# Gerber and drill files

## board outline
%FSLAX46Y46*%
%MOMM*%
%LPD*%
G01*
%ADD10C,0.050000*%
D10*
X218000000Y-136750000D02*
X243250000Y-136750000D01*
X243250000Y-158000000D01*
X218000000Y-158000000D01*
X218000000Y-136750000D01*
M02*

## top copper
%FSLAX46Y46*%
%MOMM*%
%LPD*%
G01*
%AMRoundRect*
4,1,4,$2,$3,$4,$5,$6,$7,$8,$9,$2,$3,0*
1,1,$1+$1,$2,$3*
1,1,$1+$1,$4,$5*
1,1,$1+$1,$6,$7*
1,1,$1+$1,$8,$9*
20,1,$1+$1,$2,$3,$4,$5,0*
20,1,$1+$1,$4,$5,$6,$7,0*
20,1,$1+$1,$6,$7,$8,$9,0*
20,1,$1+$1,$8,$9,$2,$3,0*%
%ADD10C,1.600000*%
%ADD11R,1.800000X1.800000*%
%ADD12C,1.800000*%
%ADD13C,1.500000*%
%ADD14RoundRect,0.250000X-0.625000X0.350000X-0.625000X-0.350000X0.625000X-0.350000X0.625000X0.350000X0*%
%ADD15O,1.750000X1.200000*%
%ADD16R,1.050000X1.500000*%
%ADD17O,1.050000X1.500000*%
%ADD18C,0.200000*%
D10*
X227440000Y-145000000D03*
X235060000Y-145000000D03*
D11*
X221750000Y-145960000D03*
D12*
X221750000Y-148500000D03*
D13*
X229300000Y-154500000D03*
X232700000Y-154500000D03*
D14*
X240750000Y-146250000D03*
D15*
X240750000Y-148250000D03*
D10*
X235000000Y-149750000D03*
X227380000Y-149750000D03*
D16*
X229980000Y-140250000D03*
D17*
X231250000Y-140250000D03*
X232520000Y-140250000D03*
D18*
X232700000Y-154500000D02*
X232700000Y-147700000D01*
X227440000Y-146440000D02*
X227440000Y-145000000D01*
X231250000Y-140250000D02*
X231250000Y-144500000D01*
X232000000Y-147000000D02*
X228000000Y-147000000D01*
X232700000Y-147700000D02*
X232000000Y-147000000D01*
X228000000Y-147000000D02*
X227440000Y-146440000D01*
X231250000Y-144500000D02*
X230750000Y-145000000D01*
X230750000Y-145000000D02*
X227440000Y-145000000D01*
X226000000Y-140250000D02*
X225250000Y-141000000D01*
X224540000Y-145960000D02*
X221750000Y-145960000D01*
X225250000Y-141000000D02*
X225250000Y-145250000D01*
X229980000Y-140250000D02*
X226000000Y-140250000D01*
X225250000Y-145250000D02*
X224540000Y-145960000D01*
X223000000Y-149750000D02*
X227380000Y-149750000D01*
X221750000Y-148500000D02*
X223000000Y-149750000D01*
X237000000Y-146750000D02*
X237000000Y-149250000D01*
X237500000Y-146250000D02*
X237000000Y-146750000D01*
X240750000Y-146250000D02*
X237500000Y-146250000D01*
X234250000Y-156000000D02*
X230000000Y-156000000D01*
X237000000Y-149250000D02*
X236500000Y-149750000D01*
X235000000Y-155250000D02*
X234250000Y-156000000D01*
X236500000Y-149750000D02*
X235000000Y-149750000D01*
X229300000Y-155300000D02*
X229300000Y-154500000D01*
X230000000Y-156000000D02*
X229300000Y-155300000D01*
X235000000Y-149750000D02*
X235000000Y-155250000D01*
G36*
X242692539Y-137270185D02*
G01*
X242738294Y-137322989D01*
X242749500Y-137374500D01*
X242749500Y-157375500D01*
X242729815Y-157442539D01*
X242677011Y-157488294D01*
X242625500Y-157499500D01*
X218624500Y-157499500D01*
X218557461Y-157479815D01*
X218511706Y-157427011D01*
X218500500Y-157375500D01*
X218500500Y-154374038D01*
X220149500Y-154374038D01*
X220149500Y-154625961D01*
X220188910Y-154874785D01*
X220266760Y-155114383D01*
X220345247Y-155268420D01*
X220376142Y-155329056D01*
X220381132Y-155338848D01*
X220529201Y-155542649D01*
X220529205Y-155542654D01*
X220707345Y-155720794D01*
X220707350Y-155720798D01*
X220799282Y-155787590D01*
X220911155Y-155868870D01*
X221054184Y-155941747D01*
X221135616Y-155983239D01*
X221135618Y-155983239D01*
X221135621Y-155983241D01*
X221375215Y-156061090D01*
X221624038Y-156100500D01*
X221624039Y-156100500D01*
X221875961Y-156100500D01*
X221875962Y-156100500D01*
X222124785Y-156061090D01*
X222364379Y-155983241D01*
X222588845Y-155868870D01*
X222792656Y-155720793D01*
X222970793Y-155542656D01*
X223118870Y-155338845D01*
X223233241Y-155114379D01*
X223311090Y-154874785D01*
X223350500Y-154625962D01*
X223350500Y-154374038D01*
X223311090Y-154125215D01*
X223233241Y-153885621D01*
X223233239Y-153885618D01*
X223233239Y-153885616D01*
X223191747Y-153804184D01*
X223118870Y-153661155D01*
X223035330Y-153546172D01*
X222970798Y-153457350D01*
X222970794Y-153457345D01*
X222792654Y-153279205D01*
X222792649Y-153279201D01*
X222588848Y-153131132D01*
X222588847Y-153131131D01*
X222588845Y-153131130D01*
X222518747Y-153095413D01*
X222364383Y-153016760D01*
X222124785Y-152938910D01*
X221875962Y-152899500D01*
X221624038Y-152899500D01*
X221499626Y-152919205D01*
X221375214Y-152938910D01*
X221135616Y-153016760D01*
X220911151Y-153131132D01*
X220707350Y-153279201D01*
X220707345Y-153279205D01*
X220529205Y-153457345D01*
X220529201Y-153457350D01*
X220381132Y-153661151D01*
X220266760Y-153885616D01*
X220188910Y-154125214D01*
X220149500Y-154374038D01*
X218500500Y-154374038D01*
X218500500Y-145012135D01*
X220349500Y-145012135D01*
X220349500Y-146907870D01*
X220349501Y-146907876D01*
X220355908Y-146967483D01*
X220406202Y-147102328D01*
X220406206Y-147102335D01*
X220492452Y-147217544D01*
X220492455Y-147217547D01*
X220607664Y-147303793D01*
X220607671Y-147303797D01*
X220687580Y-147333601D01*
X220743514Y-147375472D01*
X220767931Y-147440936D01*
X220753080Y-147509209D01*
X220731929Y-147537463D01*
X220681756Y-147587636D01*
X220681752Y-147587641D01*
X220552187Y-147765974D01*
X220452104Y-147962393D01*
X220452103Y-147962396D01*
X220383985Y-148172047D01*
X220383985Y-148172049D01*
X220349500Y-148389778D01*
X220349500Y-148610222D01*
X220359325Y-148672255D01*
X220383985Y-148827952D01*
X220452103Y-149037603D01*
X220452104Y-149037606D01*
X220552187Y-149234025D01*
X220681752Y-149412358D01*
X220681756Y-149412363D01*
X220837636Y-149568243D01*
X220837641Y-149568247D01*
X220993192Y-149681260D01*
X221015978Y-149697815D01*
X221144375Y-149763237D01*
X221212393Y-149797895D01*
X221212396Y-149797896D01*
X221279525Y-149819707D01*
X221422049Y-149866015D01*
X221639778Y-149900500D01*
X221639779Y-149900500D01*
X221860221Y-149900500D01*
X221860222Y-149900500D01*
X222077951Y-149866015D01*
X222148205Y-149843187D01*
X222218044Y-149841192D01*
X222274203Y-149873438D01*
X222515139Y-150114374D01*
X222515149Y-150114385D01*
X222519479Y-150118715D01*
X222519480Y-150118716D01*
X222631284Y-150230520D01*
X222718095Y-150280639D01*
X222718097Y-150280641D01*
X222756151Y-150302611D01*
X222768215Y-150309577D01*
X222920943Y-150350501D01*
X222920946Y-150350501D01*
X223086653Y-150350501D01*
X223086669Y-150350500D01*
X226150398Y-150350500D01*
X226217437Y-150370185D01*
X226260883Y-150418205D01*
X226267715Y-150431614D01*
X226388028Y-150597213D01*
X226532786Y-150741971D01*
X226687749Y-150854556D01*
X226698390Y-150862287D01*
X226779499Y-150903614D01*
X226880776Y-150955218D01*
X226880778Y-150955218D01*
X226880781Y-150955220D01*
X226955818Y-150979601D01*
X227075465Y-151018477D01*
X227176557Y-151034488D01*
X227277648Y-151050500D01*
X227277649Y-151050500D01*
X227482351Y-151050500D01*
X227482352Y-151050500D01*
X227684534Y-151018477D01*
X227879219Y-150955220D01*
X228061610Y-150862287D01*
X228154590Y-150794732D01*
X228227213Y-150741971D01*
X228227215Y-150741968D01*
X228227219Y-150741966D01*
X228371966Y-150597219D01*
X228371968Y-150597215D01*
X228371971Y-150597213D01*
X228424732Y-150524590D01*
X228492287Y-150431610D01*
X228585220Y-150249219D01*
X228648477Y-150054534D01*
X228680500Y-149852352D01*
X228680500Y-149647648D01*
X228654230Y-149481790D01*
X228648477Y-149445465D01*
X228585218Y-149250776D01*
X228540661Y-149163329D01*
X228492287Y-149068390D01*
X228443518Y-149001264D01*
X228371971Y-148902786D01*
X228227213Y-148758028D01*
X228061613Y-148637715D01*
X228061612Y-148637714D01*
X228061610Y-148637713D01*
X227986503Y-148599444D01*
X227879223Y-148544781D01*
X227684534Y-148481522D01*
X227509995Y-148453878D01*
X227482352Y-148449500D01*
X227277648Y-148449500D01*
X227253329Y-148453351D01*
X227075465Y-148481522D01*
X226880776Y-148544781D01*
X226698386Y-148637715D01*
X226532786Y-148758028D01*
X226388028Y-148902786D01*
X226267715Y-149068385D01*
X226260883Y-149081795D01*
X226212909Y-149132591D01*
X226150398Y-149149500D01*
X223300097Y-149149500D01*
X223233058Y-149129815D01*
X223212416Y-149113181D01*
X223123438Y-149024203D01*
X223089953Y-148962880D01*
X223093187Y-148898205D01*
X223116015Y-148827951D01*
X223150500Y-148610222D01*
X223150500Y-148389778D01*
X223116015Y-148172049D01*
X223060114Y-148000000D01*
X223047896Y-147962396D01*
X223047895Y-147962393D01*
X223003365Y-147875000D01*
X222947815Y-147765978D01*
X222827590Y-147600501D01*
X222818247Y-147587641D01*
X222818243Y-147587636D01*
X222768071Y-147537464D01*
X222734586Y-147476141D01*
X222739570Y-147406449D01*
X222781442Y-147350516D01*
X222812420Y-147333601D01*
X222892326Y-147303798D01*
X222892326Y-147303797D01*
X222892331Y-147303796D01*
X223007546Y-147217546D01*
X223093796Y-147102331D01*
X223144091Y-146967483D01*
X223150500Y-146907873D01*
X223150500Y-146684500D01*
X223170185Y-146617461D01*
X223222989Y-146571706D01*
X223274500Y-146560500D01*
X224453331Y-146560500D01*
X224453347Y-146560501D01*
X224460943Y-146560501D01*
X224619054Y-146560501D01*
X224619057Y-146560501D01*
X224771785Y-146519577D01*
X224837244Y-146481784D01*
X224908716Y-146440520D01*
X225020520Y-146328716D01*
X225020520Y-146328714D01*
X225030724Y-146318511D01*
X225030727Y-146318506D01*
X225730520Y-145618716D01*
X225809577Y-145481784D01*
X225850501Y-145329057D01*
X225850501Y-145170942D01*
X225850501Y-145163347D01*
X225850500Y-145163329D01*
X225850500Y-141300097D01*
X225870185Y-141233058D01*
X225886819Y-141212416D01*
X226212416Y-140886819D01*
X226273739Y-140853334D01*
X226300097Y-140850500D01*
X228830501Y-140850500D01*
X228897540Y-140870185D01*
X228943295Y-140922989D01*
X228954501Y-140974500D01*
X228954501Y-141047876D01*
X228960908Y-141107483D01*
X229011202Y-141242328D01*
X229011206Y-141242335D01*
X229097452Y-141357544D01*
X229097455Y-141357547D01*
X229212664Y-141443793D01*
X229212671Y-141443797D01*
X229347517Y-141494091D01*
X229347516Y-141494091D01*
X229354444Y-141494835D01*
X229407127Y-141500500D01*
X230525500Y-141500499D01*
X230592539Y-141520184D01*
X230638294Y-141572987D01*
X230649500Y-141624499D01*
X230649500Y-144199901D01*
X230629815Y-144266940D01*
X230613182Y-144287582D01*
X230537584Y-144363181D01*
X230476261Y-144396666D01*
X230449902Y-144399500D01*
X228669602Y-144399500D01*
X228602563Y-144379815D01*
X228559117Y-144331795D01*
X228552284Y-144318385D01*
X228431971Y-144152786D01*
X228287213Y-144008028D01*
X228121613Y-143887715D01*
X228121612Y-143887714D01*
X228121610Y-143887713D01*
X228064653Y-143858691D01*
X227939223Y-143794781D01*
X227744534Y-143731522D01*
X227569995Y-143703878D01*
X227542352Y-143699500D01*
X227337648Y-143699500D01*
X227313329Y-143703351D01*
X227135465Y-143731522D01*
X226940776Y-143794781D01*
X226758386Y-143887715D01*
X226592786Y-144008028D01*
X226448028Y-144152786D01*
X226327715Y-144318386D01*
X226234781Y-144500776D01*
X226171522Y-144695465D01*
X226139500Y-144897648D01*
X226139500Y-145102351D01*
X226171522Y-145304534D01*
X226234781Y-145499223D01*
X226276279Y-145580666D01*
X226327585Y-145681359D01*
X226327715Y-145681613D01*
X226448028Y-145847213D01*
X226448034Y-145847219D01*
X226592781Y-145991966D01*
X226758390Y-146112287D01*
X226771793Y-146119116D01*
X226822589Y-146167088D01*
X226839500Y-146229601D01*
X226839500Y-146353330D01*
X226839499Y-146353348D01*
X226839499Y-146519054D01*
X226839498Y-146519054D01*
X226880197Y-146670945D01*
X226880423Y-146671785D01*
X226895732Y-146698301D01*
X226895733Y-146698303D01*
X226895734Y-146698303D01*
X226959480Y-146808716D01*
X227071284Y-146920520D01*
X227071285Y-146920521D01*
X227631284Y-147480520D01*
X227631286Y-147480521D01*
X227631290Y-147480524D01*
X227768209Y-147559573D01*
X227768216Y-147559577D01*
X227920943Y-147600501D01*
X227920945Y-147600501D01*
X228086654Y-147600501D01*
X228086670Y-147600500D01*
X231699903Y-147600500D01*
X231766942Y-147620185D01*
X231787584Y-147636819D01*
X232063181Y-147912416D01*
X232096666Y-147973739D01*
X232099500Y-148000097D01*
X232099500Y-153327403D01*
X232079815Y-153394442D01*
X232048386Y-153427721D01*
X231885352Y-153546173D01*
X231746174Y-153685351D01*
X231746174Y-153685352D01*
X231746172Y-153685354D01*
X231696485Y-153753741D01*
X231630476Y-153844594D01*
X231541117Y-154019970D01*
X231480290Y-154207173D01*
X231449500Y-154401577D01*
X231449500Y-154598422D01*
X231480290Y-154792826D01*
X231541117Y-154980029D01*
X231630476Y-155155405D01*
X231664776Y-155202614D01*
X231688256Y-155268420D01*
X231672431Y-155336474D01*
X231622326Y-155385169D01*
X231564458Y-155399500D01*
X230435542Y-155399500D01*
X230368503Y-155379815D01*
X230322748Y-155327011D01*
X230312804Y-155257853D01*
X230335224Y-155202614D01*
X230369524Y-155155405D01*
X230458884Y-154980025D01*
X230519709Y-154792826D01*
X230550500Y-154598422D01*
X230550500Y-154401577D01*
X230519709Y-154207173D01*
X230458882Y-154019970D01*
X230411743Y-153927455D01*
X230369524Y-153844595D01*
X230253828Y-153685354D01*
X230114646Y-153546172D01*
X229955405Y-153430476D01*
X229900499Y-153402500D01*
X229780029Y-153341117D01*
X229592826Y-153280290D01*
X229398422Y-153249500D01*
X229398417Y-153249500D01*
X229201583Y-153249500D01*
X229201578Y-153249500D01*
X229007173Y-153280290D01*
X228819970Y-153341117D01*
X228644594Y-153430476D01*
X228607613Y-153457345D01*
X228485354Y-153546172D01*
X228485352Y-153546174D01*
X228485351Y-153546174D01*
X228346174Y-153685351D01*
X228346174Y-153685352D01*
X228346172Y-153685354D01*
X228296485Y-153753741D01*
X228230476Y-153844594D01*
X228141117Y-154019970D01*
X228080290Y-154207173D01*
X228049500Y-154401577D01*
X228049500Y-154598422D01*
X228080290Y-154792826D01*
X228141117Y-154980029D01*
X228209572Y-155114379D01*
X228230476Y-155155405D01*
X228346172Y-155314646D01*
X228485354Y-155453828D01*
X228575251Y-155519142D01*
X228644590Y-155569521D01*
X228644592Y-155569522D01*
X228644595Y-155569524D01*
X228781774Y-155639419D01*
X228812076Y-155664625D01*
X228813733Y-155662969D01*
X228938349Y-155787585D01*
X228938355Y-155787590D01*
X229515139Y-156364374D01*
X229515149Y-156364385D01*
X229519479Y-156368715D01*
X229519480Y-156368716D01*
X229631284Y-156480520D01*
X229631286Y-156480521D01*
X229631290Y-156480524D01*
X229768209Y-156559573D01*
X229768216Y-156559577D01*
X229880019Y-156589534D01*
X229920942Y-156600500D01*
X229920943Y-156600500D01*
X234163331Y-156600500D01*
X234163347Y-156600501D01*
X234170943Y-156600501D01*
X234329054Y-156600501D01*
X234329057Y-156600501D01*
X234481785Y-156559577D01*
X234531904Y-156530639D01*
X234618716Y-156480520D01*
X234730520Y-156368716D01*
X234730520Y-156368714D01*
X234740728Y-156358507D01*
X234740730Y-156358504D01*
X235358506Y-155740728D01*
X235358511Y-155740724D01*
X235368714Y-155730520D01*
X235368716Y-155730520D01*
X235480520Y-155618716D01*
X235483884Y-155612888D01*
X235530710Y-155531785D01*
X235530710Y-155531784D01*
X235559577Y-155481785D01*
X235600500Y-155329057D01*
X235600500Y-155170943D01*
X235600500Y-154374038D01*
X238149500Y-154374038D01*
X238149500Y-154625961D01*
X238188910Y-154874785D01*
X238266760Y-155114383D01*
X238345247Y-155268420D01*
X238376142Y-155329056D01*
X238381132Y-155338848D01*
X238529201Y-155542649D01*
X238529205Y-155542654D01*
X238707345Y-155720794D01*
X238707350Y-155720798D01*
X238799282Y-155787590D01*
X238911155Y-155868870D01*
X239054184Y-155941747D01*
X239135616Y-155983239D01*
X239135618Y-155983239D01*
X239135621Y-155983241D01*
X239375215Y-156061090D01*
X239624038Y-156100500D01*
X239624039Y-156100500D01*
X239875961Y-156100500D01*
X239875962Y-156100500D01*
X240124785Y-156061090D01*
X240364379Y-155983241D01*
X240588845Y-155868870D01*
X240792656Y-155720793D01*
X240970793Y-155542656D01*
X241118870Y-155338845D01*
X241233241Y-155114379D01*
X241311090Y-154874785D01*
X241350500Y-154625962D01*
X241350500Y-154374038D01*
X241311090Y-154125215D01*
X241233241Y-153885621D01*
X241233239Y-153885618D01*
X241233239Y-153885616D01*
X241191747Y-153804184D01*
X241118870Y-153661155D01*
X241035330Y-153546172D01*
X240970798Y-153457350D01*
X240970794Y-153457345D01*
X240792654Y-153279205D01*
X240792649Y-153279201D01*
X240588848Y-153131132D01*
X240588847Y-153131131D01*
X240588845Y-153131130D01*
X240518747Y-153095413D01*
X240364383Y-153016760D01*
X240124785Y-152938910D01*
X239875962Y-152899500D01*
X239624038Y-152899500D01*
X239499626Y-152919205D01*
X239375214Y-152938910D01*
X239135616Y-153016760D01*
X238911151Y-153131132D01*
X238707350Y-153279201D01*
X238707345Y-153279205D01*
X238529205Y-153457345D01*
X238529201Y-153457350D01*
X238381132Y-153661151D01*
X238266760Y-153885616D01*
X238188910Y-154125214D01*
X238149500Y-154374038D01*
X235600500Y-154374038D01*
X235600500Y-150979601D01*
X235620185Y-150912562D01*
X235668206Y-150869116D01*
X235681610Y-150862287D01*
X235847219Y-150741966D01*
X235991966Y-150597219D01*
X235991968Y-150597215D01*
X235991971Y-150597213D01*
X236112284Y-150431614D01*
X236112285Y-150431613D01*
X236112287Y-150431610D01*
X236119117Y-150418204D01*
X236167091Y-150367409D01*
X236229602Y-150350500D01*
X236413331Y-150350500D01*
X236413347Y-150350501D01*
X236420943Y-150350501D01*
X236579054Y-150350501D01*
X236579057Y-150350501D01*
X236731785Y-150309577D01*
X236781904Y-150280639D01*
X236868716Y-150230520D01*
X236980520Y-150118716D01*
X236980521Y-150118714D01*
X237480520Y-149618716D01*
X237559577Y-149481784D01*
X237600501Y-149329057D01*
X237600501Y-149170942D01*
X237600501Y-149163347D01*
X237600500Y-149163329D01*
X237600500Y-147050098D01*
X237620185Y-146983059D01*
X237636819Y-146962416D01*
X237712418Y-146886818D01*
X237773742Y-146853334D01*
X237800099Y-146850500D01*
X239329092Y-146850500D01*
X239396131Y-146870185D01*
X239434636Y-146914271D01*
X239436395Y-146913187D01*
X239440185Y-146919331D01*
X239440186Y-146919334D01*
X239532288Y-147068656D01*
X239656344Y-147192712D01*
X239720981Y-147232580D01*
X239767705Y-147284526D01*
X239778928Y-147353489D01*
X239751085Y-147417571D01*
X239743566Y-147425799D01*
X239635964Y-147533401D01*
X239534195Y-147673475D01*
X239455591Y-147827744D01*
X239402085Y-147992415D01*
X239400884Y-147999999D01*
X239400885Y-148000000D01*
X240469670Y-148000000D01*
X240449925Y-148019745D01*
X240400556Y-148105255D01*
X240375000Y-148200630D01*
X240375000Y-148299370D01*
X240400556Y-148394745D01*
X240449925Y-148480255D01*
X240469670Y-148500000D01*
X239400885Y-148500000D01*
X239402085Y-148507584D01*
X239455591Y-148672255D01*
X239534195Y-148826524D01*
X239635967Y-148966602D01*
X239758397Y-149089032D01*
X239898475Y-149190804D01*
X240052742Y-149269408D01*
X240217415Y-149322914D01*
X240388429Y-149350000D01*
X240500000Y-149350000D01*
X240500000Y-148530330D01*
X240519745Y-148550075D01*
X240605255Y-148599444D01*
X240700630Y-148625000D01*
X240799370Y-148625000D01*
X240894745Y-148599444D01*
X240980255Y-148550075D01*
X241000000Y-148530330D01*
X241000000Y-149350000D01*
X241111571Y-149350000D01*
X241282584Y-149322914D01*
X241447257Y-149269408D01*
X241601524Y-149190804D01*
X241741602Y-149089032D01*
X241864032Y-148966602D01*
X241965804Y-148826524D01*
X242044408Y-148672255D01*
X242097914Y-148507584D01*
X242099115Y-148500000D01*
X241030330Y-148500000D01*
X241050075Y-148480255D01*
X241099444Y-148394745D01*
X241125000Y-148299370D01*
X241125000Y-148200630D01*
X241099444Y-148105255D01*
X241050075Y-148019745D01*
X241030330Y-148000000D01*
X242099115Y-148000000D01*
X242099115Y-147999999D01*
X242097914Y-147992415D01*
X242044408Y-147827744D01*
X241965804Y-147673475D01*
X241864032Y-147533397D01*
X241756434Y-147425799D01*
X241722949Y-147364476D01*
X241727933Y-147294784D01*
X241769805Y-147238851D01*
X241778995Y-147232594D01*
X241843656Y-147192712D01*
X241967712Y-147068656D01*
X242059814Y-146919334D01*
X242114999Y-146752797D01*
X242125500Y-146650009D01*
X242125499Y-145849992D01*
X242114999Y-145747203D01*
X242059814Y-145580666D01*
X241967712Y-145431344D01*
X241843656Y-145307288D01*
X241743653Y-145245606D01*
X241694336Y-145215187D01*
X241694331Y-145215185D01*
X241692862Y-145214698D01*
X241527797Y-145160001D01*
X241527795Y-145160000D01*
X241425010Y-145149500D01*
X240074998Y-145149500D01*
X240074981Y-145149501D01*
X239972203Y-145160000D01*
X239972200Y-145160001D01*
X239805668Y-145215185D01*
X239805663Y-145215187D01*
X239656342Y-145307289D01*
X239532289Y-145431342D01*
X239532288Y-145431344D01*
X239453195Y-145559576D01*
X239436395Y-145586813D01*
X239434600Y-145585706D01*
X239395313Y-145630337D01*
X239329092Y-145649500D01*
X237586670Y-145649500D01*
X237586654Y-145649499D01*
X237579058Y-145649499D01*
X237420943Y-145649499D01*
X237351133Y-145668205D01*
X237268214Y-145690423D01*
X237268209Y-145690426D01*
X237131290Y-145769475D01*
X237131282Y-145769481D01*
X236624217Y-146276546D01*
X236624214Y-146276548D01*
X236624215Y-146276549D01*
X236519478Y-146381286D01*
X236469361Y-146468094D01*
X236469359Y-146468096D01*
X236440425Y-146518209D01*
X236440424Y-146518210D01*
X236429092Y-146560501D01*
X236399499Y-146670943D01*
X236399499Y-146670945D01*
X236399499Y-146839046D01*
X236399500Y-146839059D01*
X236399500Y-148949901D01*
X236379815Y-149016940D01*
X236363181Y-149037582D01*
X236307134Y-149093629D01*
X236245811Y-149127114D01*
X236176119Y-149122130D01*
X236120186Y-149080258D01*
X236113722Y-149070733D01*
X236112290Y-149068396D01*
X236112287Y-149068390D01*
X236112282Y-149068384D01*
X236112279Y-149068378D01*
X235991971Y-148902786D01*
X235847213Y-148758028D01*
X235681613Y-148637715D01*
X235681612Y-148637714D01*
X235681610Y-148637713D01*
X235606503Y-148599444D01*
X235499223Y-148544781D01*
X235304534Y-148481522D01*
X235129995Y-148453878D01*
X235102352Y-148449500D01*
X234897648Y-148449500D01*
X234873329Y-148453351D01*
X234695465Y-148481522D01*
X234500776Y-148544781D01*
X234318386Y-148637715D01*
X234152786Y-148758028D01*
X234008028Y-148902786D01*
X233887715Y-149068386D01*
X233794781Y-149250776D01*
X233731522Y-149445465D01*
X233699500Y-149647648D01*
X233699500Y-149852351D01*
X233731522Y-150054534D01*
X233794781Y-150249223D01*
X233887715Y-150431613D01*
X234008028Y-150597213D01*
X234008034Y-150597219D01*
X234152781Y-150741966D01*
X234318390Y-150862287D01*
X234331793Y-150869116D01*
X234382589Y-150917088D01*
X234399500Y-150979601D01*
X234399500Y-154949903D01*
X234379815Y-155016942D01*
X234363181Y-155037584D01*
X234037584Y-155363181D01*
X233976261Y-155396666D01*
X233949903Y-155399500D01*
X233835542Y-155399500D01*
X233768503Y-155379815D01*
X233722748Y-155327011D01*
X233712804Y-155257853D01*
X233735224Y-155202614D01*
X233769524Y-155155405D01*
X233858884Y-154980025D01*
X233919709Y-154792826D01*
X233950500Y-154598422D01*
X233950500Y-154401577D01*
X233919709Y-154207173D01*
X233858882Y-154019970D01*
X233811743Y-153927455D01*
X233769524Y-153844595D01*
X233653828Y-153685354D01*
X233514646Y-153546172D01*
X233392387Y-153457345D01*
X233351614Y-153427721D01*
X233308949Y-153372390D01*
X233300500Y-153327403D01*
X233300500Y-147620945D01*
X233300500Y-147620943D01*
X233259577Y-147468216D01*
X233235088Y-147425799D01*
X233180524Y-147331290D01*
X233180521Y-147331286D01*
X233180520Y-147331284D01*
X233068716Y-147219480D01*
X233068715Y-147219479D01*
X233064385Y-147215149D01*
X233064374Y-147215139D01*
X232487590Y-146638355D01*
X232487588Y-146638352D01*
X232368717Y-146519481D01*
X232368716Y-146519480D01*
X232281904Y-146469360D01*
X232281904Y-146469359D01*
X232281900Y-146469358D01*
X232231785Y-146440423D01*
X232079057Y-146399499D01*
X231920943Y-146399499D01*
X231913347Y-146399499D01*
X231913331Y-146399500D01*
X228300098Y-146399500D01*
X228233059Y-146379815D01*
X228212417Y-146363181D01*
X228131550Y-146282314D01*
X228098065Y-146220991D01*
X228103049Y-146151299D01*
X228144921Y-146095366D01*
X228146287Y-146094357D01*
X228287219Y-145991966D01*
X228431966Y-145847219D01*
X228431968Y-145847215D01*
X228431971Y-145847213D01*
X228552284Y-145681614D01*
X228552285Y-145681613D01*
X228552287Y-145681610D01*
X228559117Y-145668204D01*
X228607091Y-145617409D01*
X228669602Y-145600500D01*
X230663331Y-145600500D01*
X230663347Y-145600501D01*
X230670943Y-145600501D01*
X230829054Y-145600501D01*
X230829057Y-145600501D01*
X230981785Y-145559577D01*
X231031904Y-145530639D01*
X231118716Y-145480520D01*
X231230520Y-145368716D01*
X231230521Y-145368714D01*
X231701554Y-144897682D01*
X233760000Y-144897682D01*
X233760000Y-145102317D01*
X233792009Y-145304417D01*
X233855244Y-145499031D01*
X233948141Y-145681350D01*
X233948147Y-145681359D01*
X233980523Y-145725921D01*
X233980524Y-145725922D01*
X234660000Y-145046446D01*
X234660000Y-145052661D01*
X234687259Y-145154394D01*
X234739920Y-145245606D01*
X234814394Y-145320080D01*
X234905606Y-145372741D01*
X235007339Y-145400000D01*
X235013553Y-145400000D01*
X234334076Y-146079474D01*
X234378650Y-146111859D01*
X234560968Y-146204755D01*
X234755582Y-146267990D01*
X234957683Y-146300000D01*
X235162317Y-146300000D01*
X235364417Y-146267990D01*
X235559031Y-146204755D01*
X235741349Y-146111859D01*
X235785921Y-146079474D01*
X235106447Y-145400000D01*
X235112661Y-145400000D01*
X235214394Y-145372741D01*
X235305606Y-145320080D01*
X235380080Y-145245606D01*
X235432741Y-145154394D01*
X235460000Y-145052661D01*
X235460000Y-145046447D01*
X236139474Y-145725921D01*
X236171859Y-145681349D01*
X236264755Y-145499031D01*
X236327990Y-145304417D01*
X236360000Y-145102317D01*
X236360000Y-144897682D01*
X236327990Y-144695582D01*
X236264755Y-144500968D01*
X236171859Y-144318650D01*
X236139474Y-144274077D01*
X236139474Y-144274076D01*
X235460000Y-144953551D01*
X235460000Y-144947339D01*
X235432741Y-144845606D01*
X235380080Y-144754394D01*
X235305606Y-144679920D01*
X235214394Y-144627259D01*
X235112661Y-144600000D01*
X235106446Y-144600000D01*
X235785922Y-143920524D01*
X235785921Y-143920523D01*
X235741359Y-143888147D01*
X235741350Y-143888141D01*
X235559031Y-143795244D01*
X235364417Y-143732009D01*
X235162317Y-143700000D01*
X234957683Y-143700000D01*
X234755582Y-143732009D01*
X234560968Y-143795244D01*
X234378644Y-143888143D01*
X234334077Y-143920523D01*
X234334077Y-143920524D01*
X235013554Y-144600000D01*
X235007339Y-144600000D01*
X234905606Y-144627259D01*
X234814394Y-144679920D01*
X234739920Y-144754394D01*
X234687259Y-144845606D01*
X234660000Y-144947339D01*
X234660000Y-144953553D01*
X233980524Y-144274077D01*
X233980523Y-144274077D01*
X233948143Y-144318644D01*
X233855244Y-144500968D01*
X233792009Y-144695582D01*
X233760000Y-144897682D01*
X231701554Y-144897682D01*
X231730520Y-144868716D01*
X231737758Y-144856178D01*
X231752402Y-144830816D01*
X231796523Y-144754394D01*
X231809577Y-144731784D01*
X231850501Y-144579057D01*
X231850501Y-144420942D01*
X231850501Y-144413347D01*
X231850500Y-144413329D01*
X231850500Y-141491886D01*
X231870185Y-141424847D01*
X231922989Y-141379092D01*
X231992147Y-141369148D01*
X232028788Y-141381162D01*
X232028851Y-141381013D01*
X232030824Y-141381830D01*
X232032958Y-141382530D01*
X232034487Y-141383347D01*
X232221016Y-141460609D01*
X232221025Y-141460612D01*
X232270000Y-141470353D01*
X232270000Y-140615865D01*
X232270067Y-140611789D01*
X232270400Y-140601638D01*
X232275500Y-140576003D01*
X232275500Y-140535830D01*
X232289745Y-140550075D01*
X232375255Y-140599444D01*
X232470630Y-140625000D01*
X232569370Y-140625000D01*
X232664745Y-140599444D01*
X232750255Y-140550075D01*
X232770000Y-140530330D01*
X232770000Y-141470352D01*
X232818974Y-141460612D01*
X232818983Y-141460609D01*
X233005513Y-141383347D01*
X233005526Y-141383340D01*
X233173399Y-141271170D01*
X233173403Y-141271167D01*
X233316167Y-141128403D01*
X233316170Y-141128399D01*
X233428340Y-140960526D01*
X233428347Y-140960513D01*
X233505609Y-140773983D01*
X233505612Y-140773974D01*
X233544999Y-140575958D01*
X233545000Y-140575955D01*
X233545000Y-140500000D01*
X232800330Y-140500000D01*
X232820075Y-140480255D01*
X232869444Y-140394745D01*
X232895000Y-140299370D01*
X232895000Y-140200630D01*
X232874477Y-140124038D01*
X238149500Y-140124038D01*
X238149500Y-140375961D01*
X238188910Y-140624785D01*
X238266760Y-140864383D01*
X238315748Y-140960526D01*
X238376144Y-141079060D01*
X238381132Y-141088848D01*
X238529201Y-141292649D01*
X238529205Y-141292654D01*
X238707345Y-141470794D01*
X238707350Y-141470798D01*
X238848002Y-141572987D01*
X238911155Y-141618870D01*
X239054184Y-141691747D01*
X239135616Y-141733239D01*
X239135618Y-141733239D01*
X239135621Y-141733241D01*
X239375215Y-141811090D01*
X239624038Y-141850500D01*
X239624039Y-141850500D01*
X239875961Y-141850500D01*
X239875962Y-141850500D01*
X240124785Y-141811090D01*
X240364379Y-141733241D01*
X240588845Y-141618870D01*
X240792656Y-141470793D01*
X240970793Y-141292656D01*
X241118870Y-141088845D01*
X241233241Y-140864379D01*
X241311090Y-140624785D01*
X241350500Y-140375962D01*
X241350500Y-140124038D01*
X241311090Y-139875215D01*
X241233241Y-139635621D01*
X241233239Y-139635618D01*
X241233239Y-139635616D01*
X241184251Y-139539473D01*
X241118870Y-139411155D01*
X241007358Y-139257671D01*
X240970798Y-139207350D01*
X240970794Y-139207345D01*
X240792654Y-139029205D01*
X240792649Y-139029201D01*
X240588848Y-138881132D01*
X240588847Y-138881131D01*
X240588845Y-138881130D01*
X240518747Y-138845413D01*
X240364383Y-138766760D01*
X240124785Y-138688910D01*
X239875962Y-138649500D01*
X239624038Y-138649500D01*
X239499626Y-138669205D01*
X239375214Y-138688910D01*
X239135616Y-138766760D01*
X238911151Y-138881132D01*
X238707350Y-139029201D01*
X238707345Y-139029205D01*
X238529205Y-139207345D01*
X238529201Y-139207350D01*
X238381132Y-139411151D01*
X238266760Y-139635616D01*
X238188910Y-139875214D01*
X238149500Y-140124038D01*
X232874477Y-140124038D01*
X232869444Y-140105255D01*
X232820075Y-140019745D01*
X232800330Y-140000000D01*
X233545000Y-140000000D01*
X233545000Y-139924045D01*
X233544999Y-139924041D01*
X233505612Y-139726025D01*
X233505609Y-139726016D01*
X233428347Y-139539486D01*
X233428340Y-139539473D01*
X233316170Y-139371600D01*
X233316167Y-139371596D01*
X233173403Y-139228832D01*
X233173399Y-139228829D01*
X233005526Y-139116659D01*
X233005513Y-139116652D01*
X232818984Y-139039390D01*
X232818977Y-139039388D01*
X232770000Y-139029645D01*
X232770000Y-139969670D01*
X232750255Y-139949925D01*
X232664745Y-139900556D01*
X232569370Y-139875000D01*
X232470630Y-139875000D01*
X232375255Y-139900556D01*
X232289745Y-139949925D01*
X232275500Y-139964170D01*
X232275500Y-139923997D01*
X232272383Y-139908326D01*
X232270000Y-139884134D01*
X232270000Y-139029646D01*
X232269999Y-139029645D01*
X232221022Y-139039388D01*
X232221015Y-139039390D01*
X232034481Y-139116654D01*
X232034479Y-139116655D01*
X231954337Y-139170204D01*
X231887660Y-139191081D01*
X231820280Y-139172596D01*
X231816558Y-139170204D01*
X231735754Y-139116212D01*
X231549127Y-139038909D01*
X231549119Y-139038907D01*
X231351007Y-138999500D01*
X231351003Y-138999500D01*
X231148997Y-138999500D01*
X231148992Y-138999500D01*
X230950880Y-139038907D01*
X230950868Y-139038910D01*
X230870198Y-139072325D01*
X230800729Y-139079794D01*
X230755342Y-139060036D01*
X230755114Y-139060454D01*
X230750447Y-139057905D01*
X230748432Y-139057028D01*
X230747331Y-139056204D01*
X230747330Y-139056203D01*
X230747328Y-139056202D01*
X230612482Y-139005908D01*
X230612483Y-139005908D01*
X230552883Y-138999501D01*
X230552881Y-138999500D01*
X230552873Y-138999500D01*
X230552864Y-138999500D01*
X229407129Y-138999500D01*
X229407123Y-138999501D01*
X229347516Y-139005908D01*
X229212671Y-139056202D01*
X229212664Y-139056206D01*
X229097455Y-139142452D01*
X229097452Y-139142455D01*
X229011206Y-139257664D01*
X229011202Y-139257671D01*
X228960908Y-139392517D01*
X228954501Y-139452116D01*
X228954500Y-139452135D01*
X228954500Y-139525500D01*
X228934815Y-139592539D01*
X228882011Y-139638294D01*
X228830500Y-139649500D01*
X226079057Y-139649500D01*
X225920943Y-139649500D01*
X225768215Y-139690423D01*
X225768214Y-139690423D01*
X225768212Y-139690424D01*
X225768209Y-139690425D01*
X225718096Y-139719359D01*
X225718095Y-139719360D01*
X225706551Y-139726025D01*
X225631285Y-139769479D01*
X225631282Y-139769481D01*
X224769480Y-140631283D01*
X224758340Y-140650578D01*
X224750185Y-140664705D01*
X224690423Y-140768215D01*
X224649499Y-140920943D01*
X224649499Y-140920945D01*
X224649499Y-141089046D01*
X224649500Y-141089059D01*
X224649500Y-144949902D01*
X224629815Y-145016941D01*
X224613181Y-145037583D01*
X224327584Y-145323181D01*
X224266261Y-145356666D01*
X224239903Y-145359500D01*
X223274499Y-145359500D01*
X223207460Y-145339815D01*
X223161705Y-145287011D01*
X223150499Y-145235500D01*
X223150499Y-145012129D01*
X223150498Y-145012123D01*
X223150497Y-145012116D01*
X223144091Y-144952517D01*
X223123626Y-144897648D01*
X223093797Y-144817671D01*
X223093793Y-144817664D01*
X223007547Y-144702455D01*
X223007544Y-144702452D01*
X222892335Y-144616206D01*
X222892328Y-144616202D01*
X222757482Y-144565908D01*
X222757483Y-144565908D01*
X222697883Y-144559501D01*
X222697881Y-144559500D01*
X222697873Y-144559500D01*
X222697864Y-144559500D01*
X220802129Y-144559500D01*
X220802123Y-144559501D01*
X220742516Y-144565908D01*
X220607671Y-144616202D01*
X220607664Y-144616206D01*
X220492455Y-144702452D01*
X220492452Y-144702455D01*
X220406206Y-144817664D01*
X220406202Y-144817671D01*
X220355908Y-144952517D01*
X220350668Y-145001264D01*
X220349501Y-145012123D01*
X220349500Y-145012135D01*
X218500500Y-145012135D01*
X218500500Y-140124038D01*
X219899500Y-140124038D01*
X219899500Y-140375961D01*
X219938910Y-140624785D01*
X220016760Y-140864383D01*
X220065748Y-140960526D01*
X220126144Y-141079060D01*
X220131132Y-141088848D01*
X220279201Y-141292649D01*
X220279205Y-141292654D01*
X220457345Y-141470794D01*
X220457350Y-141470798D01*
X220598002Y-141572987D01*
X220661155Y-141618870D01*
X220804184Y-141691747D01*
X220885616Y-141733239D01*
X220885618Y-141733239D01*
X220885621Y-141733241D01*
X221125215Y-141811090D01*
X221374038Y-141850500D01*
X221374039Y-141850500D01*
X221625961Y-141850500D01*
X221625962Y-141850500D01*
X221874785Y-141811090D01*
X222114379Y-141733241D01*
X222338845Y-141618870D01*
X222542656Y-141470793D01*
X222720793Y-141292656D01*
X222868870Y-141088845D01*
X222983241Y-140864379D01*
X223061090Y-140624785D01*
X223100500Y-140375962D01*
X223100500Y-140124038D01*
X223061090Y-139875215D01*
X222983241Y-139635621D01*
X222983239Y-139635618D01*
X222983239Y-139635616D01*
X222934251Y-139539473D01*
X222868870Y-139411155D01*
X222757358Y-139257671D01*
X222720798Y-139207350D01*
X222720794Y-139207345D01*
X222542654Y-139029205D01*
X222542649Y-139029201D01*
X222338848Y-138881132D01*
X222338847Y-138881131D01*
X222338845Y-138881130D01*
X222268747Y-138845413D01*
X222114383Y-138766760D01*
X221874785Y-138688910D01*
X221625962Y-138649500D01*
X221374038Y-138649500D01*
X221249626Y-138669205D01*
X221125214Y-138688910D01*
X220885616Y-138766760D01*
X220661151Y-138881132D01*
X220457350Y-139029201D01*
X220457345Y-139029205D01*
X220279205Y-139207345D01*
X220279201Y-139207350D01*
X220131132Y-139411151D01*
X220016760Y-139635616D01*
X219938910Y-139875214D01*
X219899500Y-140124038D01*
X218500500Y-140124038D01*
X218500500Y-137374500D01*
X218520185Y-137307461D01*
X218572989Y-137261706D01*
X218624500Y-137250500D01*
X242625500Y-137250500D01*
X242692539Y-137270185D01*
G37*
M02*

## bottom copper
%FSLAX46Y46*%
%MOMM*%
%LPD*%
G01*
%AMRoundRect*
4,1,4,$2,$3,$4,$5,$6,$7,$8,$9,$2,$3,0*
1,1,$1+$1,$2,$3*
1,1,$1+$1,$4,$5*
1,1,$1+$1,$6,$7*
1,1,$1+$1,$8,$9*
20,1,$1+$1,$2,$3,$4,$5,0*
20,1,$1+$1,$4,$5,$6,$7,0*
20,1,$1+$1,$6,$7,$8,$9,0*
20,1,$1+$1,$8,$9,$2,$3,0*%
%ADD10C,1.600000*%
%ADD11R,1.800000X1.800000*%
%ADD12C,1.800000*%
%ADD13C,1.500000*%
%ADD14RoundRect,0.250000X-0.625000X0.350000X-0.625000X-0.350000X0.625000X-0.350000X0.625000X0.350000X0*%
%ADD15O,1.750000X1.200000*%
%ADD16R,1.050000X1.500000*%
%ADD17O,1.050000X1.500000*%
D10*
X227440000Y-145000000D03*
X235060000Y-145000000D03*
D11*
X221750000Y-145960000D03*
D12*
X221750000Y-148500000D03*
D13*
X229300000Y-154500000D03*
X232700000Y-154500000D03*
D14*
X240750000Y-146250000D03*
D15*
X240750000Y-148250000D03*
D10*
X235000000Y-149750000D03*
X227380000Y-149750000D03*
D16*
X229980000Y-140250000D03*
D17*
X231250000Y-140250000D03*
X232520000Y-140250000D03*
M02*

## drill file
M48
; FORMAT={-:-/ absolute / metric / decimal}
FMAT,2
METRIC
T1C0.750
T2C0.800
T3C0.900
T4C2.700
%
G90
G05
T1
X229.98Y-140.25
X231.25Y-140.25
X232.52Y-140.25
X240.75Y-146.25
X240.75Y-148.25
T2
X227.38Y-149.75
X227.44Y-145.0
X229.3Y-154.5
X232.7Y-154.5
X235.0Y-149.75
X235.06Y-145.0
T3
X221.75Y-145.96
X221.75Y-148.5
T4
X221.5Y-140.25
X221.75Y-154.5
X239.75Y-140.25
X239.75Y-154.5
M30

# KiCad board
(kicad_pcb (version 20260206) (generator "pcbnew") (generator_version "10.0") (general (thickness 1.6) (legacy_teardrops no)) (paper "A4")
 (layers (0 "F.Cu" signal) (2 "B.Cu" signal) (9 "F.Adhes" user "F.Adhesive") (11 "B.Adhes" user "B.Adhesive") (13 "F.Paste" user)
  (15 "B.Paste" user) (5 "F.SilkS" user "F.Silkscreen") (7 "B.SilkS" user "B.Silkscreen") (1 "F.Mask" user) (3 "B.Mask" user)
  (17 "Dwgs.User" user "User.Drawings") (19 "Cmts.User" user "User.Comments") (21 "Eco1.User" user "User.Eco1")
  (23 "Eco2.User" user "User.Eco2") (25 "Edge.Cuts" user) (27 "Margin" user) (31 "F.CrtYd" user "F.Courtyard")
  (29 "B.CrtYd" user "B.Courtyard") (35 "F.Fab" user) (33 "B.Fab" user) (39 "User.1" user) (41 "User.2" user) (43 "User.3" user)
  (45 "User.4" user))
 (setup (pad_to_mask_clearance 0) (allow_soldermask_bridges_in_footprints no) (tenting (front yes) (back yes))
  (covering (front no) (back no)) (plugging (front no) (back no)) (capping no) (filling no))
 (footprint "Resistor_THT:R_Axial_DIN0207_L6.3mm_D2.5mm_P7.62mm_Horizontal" (layer "F.Cu") (at 227.44 145)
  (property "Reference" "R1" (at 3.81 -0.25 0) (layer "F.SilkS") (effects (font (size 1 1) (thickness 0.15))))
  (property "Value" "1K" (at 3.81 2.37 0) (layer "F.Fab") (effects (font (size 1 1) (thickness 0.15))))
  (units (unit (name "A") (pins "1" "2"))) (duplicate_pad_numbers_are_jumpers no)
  (pad "1" thru_hole circle (at 0 0) (size 1.6 1.6) (drill 0.8) (layers "*.Cu" "*.Mask") (remove_unused_layers no) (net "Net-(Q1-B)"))
  (pad "2" thru_hole circle (at 7.62 0) (size 1.6 1.6) (drill 0.8) (layers "*.Cu" "*.Mask") (remove_unused_layers no) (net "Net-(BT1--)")))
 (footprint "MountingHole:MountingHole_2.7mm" (layer "F.Cu") (at 221.5 140.25)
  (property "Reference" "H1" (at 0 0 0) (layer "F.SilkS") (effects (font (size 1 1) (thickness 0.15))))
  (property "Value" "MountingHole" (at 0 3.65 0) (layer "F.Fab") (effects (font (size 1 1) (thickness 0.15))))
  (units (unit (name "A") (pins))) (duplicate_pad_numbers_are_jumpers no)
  (pad "" np_thru_hole circle (at 0 0) (size 2.7 2.7) (drill 2.7) (layers "*.Cu" "*.Mask")))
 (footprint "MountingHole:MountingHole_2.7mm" (layer "F.Cu") (at 221.75 154.5)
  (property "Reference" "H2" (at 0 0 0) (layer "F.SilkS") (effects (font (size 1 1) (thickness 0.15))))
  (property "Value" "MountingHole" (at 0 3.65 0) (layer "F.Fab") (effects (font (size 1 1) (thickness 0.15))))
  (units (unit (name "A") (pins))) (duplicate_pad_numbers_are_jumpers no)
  (pad "" np_thru_hole circle (at 0 0) (size 2.7 2.7) (drill 2.7) (layers "*.Cu" "*.Mask")))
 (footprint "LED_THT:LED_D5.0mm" (layer "F.Cu") (at 221.75 145.96 -90)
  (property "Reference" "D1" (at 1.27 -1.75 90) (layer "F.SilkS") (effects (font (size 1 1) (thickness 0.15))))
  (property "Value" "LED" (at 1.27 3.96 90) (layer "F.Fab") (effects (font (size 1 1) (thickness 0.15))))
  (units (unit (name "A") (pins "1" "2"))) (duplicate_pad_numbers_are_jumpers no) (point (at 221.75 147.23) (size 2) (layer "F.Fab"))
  (pad "1" thru_hole rect (at 0 0 270) (size 1.8 1.8) (drill 0.9) (layers "*.Cu" "*.Mask") (remove_unused_layers no) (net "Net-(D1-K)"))
  (pad "2" thru_hole circle (at 2.54 0 270) (size 1.8 1.8) (drill 0.9) (layers "*.Cu" "*.Mask") (remove_unused_layers no) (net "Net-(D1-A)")))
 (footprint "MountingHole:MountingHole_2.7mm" (layer "F.Cu") (at 239.75 140.25)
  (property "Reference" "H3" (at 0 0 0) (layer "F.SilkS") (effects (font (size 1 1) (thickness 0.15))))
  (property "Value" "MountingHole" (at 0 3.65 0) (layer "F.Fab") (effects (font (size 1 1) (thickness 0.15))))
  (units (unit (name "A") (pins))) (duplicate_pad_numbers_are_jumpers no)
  (pad "" np_thru_hole circle (at 0 0) (size 2.7 2.7) (drill 2.7) (layers "*.Cu" "*.Mask")))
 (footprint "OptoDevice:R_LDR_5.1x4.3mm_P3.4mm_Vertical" (layer "F.Cu") (at 229.3 154.5)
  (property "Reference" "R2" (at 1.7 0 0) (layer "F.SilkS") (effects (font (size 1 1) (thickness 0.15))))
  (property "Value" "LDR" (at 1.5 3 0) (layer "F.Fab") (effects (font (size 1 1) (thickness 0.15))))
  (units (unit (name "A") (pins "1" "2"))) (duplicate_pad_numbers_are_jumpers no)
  (pad "1" thru_hole circle (at 0 0) (size 1.5 1.5) (drill 0.8) (layers "*.Cu" "*.Mask") (remove_unused_layers no) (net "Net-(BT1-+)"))
  (pad "2" thru_hole circle (at 3.4 0) (size 1.5 1.5) (drill 0.8) (layers "*.Cu" "*.Mask") (remove_unused_layers no) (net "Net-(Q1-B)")))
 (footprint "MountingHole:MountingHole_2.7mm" (layer "F.Cu") (at 239.75 154.5)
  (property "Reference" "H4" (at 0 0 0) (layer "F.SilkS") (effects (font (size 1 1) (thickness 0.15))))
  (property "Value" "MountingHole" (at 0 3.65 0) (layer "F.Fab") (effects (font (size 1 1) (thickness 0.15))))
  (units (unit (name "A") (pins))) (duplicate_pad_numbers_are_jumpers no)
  (pad "" np_thru_hole circle (at 0 0) (size 2.7 2.7) (drill 2.7) (layers "*.Cu" "*.Mask")))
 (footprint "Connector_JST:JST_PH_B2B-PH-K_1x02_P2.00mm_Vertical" (layer "F.Cu") (at 240.75 146.25 -90)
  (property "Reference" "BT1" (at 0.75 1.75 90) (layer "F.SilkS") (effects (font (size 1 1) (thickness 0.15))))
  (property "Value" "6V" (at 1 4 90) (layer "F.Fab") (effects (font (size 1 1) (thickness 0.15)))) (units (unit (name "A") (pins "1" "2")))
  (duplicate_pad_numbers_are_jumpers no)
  (pad "1" thru_hole roundrect (at 0 0 270) (size 1.2 1.75) (drill 0.75) (layers "*.Cu" "*.Mask") (remove_unused_layers no)
   (roundrect_rratio 0.208333) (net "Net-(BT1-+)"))
  (pad "2" thru_hole oval (at 2 0 270) (size 1.2 1.75) (drill 0.75) (layers "*.Cu" "*.Mask") (remove_unused_layers no) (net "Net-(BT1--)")))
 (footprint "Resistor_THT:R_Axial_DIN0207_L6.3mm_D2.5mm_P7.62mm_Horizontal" (layer "F.Cu") (at 235 149.75 180)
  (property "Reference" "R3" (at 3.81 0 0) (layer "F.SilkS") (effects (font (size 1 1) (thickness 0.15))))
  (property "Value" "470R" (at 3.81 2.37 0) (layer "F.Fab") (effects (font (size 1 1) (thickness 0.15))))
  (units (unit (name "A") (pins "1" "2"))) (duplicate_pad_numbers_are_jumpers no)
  (pad "1" thru_hole circle (at 0 0 180) (size 1.6 1.6) (drill 0.8) (layers "*.Cu" "*.Mask") (remove_unused_layers no) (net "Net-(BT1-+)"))
  (pad "2" thru_hole circle (at 7.62 0 180) (size 1.6 1.6) (drill 0.8) (layers "*.Cu" "*.Mask") (remove_unused_layers no) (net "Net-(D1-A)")))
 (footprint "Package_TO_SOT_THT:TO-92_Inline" (layer "F.Cu") (at 229.98 140.25)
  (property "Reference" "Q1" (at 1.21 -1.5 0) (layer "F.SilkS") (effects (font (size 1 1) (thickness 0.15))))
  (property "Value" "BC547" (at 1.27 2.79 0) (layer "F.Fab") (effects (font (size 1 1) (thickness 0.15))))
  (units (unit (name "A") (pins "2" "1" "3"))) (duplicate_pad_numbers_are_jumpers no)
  (pad "1" thru_hole rect (at 0 0) (size 1.05 1.5) (drill 0.75) (layers "*.Cu" "*.Mask") (remove_unused_layers no) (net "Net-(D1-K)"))
  (pad "2" thru_hole oval (at 1.27 0) (size 1.05 1.5) (drill 0.75) (layers "*.Cu" "*.Mask") (remove_unused_layers no) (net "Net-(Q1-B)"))
  (pad "3" thru_hole oval (at 2.54 0) (size 1.05 1.5) (drill 0.75) (layers "*.Cu" "*.Mask") (remove_unused_layers no) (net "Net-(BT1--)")))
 (gr_rect (start 218 136.75) (end 243.25 158) (stroke (width 0.05) (type default)) (fill no) (layer "Edge.Cuts"))
 (segment (start 232.7 154.5) (end 232.7 147.7) (width 0.2) (layer "F.Cu") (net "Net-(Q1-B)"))
 (segment (start 227.44 146.44) (end 227.44 145) (width 0.2) (layer "F.Cu") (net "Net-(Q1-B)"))
 (segment (start 231.25 140.25) (end 231.25 144.5) (width 0.2) (layer "F.Cu") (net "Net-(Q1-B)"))
 (segment (start 232 147) (end 228 147) (width 0.2) (layer "F.Cu") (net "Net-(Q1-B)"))
 (segment (start 232.7 147.7) (end 232 147) (width 0.2) (layer "F.Cu") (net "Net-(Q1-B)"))
 (segment (start 228 147) (end 227.44 146.44) (width 0.2) (layer "F.Cu") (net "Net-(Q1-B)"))
 (segment (start 231.25 144.5) (end 230.75 145) (width 0.2) (layer "F.Cu") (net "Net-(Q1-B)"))
 (segment (start 230.75 145) (end 227.44 145) (width 0.2) (layer "F.Cu") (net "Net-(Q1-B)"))
 (segment (start 226 140.25) (end 225.25 141) (width 0.2) (layer "F.Cu") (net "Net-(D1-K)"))
 (segment (start 224.54 145.96) (end 221.75 145.96) (width 0.2) (layer "F.Cu") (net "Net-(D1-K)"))
 (segment (start 225.25 141) (end 225.25 145.25) (width 0.2) (layer "F.Cu") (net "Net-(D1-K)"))
 (segment (start 229.98 140.25) (end 226 140.25) (width 0.2) (layer "F.Cu") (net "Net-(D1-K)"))
 (segment (start 225.25 145.25) (end 224.54 145.96) (width 0.2) (layer "F.Cu") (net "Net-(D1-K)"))
 (segment (start 223 149.75) (end 227.38 149.75) (width 0.2) (layer "F.Cu") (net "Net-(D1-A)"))
 (segment (start 221.75 148.5) (end 223 149.75) (width 0.2) (layer "F.Cu") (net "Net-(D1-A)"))
 (segment (start 237 146.75) (end 237 149.25) (width 0.2) (layer "F.Cu") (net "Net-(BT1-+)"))
 (segment (start 237.5 146.25) (end 237 146.75) (width 0.2) (layer "F.Cu") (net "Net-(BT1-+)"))
 (segment (start 240.75 146.25) (end 237.5 146.25) (width 0.2) (layer "F.Cu") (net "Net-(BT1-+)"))
 (segment (start 234.25 156) (end 230 156) (width 0.2) (layer "F.Cu") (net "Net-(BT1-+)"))
 (segment (start 237 149.25) (end 236.5 149.75) (width 0.2) (layer "F.Cu") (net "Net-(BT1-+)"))
 (segment (start 235 155.25) (end 234.25 156) (width 0.2) (layer "F.Cu") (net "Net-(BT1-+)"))
 (segment (start 236.5 149.75) (end 235 149.75) (width 0.2) (layer "F.Cu") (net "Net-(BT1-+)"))
 (segment (start 229.3 155.3) (end 229.3 154.5) (width 0.2) (layer "F.Cu") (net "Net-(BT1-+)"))
 (segment (start 230 156) (end 229.3 155.3) (width 0.2) (layer "F.Cu") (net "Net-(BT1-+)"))
 (segment (start 235 149.75) (end 235 155.25) (width 0.2) (layer "F.Cu") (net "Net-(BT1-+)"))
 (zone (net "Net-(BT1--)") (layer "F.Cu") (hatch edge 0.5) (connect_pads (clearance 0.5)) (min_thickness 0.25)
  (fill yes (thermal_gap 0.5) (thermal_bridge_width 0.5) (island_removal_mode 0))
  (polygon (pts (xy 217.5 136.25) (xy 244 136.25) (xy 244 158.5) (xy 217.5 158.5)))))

